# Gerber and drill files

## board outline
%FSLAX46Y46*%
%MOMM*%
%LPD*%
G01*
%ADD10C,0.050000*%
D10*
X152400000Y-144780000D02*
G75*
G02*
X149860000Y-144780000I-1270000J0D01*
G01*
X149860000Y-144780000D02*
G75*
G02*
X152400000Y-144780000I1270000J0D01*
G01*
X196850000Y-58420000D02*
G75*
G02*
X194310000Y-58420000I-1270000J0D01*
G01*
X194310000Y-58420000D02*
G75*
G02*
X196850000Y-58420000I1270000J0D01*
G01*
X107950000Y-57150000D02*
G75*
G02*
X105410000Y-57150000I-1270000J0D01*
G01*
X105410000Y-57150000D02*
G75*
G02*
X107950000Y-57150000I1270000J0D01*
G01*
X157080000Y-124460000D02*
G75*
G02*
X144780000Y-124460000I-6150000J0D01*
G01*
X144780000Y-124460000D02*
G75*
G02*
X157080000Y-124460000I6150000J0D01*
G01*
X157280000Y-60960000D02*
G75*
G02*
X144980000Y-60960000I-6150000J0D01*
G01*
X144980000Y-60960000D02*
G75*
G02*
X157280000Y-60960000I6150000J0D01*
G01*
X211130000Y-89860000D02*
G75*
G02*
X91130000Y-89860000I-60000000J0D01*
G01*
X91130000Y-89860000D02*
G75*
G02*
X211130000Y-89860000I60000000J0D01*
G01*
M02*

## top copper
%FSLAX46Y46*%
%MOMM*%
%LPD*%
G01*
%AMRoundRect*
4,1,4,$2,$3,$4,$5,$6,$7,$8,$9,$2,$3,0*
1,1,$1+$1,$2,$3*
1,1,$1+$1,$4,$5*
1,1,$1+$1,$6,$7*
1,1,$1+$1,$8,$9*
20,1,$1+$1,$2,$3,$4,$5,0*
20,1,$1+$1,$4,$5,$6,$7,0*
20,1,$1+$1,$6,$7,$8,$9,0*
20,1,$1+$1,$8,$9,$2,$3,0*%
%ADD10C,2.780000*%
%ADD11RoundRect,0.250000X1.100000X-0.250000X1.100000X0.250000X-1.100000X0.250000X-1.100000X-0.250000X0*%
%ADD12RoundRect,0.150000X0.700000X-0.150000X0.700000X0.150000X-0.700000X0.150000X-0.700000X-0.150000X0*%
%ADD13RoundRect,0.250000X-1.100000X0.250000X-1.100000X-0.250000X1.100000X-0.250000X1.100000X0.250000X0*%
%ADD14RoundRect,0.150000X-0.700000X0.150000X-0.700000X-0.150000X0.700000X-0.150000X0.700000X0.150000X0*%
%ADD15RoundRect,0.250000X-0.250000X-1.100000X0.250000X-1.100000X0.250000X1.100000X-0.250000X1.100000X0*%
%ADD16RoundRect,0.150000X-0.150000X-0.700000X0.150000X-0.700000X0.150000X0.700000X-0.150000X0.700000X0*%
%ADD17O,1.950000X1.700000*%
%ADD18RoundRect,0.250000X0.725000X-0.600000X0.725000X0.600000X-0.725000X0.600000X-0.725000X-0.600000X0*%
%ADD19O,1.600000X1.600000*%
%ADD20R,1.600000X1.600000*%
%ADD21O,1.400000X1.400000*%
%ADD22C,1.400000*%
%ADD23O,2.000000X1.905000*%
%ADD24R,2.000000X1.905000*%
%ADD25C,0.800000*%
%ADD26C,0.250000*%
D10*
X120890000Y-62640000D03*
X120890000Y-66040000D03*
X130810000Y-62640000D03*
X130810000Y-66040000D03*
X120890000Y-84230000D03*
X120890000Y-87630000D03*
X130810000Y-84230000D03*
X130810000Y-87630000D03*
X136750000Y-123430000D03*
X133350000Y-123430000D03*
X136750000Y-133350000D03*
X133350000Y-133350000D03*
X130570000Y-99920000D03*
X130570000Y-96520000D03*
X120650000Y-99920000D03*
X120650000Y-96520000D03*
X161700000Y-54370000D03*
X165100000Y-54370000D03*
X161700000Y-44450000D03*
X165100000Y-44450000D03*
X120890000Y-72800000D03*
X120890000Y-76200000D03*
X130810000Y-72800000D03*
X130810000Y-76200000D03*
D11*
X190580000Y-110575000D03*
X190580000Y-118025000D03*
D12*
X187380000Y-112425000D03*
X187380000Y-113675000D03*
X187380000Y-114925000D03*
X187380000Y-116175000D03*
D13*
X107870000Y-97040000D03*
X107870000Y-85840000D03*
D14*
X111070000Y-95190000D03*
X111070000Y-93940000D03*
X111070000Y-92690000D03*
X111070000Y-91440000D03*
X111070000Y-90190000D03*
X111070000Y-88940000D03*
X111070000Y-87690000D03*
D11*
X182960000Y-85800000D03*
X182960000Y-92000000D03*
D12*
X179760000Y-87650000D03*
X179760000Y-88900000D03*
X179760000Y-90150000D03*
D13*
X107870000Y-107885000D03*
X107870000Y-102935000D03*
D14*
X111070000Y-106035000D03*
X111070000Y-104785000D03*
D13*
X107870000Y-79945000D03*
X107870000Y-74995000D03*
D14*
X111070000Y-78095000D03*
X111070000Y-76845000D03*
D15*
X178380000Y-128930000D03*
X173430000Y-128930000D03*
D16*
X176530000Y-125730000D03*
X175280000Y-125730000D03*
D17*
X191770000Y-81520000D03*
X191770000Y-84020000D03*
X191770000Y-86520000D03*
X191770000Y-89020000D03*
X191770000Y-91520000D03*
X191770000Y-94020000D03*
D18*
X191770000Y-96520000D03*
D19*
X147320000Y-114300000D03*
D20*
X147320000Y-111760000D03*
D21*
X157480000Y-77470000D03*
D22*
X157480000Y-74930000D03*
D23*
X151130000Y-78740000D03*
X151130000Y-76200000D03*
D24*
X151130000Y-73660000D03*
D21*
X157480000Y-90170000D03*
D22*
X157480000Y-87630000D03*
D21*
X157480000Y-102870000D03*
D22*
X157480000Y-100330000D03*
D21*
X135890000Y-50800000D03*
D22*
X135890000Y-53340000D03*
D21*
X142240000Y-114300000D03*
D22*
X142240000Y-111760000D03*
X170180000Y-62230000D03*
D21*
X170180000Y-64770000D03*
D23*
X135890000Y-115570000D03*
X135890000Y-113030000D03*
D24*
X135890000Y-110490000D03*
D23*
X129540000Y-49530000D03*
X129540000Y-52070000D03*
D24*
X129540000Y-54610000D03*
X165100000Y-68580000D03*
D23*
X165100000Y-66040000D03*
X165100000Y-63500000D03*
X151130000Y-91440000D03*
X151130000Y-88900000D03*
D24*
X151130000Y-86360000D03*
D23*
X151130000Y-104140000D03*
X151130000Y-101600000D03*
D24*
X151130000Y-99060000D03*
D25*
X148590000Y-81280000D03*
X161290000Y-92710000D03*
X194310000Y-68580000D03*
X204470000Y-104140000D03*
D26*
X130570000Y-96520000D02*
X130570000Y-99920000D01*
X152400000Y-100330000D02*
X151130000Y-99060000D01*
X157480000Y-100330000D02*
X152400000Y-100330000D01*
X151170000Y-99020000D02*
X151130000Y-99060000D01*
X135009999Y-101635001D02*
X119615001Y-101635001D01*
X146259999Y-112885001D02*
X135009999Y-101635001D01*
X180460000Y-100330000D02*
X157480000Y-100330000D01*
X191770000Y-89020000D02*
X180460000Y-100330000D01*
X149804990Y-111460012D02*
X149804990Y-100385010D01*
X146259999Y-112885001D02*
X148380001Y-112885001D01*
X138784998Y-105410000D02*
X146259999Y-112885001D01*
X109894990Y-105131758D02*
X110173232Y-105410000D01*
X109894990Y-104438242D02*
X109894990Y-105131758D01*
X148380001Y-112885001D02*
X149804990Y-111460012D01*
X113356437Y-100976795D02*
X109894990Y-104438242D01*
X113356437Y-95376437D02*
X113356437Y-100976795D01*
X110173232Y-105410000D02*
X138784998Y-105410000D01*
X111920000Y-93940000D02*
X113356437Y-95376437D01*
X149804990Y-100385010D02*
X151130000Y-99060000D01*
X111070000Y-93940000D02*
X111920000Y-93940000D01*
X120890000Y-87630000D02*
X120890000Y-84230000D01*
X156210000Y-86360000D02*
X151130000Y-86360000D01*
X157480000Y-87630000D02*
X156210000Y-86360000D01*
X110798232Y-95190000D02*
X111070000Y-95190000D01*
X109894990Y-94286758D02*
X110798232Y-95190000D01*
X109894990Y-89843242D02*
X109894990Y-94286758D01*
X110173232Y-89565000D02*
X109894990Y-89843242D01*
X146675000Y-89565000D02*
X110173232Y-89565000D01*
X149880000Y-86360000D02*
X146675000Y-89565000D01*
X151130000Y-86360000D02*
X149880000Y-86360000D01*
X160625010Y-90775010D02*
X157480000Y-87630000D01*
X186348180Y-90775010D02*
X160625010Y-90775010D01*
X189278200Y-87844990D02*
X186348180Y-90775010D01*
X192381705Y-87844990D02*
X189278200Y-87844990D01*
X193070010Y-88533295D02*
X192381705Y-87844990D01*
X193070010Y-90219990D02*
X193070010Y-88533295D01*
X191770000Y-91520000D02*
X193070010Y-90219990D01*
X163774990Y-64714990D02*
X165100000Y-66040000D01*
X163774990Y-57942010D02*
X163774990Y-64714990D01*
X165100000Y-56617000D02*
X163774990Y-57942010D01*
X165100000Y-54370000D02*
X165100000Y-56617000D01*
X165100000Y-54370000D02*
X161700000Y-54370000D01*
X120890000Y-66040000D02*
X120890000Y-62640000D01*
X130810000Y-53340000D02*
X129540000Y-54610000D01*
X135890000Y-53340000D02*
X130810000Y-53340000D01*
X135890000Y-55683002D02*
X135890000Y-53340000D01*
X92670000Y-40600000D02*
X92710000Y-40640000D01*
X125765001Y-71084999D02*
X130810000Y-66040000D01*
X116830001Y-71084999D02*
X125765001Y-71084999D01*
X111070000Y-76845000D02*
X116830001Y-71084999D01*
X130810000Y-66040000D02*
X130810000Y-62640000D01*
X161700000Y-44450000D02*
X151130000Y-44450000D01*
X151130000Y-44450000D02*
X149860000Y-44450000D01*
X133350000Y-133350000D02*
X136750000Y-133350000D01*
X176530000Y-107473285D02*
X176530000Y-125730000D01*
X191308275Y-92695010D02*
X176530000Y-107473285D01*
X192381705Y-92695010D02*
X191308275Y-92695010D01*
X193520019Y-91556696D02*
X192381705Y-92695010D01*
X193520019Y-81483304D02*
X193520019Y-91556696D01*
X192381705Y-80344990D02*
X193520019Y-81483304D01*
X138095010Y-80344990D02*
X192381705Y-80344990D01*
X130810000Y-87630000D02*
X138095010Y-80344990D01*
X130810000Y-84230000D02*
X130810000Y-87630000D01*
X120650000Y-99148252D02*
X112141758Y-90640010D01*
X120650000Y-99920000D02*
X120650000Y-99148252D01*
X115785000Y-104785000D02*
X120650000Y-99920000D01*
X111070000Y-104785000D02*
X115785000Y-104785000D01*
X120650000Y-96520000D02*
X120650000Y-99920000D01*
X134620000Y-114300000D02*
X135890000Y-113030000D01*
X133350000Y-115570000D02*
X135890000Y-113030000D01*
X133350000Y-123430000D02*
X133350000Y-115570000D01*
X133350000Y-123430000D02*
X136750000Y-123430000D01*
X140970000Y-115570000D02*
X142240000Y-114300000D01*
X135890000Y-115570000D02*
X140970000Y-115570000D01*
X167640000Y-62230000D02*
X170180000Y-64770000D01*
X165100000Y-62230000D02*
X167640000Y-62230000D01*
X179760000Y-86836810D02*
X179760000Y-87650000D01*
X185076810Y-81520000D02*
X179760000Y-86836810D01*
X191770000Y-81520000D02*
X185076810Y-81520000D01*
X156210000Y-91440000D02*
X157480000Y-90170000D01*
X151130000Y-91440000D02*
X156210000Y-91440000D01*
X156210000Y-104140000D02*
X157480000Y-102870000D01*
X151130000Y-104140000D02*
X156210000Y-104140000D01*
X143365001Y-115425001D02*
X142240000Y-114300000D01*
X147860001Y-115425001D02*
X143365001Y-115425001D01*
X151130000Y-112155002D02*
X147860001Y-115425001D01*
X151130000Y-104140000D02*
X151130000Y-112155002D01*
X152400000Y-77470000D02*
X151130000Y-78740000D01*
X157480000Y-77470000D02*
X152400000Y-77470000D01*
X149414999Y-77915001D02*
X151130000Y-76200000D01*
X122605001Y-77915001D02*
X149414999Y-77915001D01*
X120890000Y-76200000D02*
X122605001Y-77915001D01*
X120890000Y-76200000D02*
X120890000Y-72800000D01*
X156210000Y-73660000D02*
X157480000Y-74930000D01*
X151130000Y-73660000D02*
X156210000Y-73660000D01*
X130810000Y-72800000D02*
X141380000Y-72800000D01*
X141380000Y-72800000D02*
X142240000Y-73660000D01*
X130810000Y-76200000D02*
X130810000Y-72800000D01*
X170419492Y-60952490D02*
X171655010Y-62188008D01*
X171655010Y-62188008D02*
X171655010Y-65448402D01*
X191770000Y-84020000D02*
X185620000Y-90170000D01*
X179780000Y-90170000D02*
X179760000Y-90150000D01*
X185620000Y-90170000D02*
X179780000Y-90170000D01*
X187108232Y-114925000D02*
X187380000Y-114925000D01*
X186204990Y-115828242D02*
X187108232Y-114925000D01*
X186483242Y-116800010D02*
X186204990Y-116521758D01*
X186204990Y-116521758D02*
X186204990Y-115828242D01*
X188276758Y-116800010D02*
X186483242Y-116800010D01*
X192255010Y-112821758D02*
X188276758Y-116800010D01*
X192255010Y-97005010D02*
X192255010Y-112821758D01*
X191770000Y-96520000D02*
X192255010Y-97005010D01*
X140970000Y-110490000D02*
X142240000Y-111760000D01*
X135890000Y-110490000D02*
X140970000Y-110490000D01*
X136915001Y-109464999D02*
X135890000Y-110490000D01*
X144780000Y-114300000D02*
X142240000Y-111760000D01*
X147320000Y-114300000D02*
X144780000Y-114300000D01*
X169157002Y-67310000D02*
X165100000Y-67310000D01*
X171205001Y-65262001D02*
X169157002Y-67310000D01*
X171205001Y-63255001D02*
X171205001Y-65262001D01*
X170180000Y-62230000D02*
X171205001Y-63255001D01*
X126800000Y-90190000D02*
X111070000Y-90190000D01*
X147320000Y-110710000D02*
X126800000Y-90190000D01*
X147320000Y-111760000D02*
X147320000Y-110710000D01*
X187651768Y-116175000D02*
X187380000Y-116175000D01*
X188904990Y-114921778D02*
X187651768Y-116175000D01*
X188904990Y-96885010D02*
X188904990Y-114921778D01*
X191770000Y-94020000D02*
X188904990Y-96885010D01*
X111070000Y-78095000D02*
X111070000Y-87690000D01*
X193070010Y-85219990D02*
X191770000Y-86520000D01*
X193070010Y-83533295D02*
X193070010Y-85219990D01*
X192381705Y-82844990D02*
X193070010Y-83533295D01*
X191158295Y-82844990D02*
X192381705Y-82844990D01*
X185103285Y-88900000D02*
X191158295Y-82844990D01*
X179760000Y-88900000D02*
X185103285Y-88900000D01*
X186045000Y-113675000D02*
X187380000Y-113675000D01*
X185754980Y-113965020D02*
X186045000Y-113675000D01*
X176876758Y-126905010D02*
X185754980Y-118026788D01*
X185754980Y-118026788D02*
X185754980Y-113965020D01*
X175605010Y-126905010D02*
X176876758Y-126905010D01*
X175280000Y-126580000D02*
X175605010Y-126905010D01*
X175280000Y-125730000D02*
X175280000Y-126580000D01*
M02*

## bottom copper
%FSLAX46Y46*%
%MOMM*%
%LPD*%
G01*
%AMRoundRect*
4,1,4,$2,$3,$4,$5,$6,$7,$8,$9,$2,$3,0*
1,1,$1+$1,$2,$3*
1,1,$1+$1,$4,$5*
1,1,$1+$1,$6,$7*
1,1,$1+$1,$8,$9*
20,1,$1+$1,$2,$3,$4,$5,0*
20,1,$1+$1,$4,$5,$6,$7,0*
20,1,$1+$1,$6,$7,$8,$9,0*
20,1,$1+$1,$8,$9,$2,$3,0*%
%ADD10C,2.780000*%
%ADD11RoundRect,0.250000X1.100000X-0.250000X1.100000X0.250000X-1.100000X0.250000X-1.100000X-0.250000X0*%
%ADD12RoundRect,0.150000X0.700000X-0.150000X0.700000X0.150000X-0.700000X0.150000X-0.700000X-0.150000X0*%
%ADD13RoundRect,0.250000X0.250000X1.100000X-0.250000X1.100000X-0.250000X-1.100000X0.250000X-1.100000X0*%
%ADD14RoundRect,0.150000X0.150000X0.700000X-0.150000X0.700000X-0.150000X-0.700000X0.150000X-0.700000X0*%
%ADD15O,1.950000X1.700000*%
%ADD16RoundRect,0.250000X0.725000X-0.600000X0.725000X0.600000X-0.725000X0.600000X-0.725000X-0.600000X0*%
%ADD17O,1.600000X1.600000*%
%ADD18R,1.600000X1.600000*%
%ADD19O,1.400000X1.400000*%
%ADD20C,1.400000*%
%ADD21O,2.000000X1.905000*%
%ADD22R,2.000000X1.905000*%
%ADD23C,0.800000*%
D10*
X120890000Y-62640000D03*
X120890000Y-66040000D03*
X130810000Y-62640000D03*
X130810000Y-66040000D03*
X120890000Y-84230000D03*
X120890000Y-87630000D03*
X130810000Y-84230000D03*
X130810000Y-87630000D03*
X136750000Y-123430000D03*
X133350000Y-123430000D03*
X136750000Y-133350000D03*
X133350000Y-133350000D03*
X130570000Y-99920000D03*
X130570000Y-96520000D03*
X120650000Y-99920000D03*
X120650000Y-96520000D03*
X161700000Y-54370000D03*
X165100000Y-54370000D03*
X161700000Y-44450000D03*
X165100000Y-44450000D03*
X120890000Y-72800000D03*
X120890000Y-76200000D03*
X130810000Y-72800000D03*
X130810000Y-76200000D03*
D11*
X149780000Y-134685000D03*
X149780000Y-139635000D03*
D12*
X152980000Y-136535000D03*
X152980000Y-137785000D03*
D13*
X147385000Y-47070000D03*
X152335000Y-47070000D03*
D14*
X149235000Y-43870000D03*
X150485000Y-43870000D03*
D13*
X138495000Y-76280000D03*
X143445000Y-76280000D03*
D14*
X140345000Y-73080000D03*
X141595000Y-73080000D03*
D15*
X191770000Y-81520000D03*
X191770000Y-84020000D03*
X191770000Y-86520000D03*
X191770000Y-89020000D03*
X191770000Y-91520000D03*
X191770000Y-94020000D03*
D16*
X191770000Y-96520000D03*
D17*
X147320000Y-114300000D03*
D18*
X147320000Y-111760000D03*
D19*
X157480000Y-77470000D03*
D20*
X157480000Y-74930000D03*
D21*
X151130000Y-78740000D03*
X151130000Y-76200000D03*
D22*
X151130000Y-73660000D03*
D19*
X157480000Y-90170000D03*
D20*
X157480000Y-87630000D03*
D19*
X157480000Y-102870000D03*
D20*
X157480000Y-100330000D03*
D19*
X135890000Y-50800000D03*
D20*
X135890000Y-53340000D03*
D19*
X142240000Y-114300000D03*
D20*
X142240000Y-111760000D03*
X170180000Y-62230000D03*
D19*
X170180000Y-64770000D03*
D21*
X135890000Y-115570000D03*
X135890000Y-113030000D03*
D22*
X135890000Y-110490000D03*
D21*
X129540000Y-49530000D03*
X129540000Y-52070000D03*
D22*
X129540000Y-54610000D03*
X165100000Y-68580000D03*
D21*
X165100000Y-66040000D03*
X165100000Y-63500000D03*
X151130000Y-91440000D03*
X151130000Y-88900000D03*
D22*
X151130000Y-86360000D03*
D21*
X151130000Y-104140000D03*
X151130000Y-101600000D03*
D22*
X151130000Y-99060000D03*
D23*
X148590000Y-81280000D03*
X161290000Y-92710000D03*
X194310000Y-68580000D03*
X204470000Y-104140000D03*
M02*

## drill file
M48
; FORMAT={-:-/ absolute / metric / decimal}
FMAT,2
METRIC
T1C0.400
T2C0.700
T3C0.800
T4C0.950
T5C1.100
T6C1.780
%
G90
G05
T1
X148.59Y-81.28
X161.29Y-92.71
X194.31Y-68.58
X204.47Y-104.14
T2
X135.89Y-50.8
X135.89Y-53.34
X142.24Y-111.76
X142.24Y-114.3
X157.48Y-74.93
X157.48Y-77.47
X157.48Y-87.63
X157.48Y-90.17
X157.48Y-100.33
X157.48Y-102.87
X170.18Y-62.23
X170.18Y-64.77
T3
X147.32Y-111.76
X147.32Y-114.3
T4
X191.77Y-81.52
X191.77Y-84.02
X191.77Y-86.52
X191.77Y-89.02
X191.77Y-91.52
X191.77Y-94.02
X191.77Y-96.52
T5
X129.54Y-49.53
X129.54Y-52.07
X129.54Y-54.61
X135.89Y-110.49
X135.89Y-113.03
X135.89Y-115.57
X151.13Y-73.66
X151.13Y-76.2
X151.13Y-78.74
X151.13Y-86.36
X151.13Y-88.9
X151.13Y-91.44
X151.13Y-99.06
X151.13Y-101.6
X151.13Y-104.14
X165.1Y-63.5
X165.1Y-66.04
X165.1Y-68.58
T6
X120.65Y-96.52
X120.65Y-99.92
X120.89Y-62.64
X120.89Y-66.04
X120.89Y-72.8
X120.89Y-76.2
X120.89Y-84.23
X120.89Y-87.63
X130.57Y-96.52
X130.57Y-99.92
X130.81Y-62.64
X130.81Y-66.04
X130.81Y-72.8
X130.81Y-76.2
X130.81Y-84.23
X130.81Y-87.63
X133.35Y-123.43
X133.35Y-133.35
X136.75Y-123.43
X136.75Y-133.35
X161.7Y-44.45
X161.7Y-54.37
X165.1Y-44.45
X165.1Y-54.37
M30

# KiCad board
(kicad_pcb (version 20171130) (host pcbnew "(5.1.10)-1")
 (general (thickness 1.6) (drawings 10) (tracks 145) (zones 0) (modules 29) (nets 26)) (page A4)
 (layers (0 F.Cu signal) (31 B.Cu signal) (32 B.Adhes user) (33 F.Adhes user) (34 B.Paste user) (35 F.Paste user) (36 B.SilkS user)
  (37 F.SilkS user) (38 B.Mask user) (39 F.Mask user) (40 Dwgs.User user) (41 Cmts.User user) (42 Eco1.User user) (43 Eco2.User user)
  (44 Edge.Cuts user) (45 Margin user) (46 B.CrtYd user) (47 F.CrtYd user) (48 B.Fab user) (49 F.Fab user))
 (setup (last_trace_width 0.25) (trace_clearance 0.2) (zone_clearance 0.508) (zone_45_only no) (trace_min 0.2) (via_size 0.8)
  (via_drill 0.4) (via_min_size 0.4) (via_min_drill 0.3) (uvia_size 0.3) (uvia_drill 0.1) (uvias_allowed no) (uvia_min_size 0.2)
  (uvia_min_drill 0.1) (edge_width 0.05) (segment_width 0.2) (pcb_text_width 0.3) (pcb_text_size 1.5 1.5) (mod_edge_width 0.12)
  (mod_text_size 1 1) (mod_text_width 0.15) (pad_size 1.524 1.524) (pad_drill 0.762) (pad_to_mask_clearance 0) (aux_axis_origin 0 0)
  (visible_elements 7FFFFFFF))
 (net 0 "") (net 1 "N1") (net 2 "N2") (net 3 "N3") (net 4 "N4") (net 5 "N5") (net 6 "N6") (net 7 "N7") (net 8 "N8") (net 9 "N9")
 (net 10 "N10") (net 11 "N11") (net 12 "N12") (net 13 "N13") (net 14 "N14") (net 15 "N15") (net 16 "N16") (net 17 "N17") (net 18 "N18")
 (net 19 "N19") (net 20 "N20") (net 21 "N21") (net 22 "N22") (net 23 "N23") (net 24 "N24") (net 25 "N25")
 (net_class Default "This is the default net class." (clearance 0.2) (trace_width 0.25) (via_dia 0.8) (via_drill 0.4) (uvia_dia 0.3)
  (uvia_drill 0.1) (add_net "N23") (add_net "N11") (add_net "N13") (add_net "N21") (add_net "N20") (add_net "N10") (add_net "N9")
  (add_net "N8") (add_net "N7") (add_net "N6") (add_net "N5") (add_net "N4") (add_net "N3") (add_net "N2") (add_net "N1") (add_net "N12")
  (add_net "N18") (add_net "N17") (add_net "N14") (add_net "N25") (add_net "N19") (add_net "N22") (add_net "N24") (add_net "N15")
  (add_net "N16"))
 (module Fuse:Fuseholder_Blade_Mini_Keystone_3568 (layer F.Cu) (at 130.81 66.04 180)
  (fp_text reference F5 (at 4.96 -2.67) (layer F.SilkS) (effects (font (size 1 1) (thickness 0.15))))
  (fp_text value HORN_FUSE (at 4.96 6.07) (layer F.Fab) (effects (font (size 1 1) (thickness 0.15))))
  (pad 2 thru_hole circle (at 9.92 3.4 180) (size 2.78 2.78) (drill 1.78) (layers *.Cu *.Mask) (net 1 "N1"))
  (pad 2 thru_hole circle (at 9.92 0 180) (size 2.78 2.78) (drill 1.78) (layers *.Cu *.Mask) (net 1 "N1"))
  (pad 1 thru_hole circle (at 0 3.4 180) (size 2.78 2.78) (drill 1.78) (layers *.Cu *.Mask) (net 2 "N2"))
  (pad 1 thru_hole circle (at 0 0 180) (size 2.78 2.78) (drill 1.78) (layers *.Cu *.Mask) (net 2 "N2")))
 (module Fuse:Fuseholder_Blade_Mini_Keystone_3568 (layer F.Cu) (at 130.81 87.63 180)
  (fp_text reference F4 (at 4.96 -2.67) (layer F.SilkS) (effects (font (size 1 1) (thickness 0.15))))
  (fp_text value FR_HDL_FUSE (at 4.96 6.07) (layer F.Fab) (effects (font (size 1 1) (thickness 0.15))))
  (pad 2 thru_hole circle (at 9.92 3.4 180) (size 2.78 2.78) (drill 1.78) (layers *.Cu *.Mask) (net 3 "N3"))
  (pad 2 thru_hole circle (at 9.92 0 180) (size 2.78 2.78) (drill 1.78) (layers *.Cu *.Mask) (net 3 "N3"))
  (pad 1 thru_hole circle (at 0 3.4 180) (size 2.78 2.78) (drill 1.78) (layers *.Cu *.Mask) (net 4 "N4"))
  (pad 1 thru_hole circle (at 0 0 180) (size 2.78 2.78) (drill 1.78) (layers *.Cu *.Mask) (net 4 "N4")))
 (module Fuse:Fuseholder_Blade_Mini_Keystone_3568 (layer F.Cu) (at 133.35 133.35 90)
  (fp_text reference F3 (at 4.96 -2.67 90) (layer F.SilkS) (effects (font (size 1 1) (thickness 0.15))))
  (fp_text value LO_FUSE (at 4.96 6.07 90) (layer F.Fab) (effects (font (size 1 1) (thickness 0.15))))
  (pad 2 thru_hole circle (at 9.92 3.4 90) (size 2.78 2.78) (drill 1.78) (layers *.Cu *.Mask) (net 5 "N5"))
  (pad 2 thru_hole circle (at 9.92 0 90) (size 2.78 2.78) (drill 1.78) (layers *.Cu *.Mask) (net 5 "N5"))
  (pad 1 thru_hole circle (at 0 3.4 90) (size 2.78 2.78) (drill 1.78) (layers *.Cu *.Mask) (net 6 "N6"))
  (pad 1 thru_hole circle (at 0 0 90) (size 2.78 2.78) (drill 1.78) (layers *.Cu *.Mask) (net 6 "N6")))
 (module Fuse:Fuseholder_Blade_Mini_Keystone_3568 (layer F.Cu) (at 120.65 96.52)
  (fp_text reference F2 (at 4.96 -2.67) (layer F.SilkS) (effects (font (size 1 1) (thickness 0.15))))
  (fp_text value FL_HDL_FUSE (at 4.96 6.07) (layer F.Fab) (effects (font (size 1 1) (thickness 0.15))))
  (pad 2 thru_hole circle (at 9.92 3.4) (size 2.78 2.78) (drill 1.78) (layers *.Cu *.Mask) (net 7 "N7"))
  (pad 2 thru_hole circle (at 9.92 0) (size 2.78 2.78) (drill 1.78) (layers *.Cu *.Mask) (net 7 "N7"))
  (pad 1 thru_hole circle (at 0 3.4) (size 2.78 2.78) (drill 1.78) (layers *.Cu *.Mask) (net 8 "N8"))
  (pad 1 thru_hole circle (at 0 0) (size 2.78 2.78) (drill 1.78) (layers *.Cu *.Mask) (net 8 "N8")))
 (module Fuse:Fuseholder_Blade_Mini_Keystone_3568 (layer F.Cu) (at 165.1 44.45 270)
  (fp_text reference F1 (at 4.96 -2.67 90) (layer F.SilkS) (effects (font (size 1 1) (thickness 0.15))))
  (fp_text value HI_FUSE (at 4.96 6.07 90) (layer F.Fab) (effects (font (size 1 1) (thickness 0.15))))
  (pad 2 thru_hole circle (at 9.92 3.4 270) (size 2.78 2.78) (drill 1.78) (layers *.Cu *.Mask) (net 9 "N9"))
  (pad 2 thru_hole circle (at 9.92 0 270) (size 2.78 2.78) (drill 1.78) (layers *.Cu *.Mask) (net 9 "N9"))
  (pad 1 thru_hole circle (at 0 3.4 270) (size 2.78 2.78) (drill 1.78) (layers *.Cu *.Mask) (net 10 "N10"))
  (pad 1 thru_hole circle (at 0 0 270) (size 2.78 2.78) (drill 1.78) (layers *.Cu *.Mask) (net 10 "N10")))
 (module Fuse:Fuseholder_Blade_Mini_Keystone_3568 (layer F.Cu) (at 130.81 76.2 180)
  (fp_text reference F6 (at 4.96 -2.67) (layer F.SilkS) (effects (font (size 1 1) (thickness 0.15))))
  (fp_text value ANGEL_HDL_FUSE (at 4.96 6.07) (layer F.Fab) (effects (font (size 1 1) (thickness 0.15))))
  (pad 2 thru_hole circle (at 9.92 3.4 180) (size 2.78 2.78) (drill 1.78) (layers *.Cu *.Mask) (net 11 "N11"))
  (pad 2 thru_hole circle (at 9.92 0 180) (size 2.78 2.78) (drill 1.78) (layers *.Cu *.Mask) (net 11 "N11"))
  (pad 1 thru_hole circle (at 0 3.4 180) (size 2.78 2.78) (drill 1.78) (layers *.Cu *.Mask) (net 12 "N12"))
  (pad 1 thru_hole circle (at 0 0 180) (size 2.78 2.78) (drill 1.78) (layers *.Cu *.Mask) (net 12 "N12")))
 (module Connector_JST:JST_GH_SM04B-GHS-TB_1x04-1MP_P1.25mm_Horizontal (layer F.Cu) (at 189.23 114.3 90)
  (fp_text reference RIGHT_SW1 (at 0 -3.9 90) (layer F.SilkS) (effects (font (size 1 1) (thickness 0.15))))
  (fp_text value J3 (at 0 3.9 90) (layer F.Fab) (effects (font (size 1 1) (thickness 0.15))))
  (pad MP smd roundrect (at 3.725 1.35 90) (size 1 2.7) (layers F.Cu F.Paste F.Mask) (roundrect_rratio 0.25))
  (pad MP smd roundrect (at -3.725 1.35 90) (size 1 2.7) (layers F.Cu F.Paste F.Mask) (roundrect_rratio 0.25))
  (pad 4 smd roundrect (at 1.875 -1.85 90) (size 0.6 1.7) (layers F.Cu F.Paste F.Mask) (roundrect_rratio 0.25) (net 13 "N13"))
  (pad 3 smd roundrect (at 0.625 -1.85 90) (size 0.6 1.7) (layers F.Cu F.Paste F.Mask) (roundrect_rratio 0.25) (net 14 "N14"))
  (pad 2 smd roundrect (at -0.625 -1.85 90) (size 0.6 1.7) (layers F.Cu F.Paste F.Mask) (roundrect_rratio 0.25) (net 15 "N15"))
  (pad 1 smd roundrect (at -1.875 -1.85 90) (size 0.6 1.7) (layers F.Cu F.Paste F.Mask) (roundrect_rratio 0.25) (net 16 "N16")))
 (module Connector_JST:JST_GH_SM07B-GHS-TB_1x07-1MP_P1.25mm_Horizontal (layer F.Cu) (at 109.22 91.44 270)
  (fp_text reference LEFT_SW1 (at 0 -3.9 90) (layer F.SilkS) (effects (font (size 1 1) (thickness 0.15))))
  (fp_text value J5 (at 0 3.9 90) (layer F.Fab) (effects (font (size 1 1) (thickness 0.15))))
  (pad MP smd roundrect (at 5.6 1.35 270) (size 1 2.7) (layers F.Cu F.Paste F.Mask) (roundrect_rratio 0.25))
  (pad MP smd roundrect (at -5.6 1.35 270) (size 1 2.7) (layers F.Cu F.Paste F.Mask) (roundrect_rratio 0.25))
  (pad 7 smd roundrect (at 3.75 -1.85 270) (size 0.6 1.7) (layers F.Cu F.Paste F.Mask) (roundrect_rratio 0.25) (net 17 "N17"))
  (pad 6 smd roundrect (at 2.5 -1.85 270) (size 0.6 1.7) (layers F.Cu F.Paste F.Mask) (roundrect_rratio 0.25) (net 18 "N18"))
  (pad 5 smd roundrect (at 1.25 -1.85 270) (size 0.6 1.7) (layers F.Cu F.Paste F.Mask) (roundrect_rratio 0.25) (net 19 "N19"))
  (pad 4 smd roundrect (at 0 -1.85 270) (size 0.6 1.7) (layers F.Cu F.Paste F.Mask) (roundrect_rratio 0.25) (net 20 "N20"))
  (pad 3 smd roundrect (at -1.25 -1.85 270) (size 0.6 1.7) (layers F.Cu F.Paste F.Mask) (roundrect_rratio 0.25) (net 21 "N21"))
  (pad 2 smd roundrect (at -2.5 -1.85 270) (size 0.6 1.7) (layers F.Cu F.Paste F.Mask) (roundrect_rratio 0.25) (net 13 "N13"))
  (pad 1 smd roundrect (at -3.75 -1.85 270) (size 0.6 1.7) (layers F.Cu F.Paste F.Mask) (roundrect_rratio 0.25) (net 14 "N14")))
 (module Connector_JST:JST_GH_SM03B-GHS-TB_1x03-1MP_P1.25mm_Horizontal (layer F.Cu) (at 181.61 88.9 90)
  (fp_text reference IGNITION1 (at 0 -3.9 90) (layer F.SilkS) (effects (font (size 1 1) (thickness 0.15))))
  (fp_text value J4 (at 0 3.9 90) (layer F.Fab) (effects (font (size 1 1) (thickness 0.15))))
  (pad MP smd roundrect (at 3.1 1.35 90) (size 1 2.7) (layers F.Cu F.Paste F.Mask) (roundrect_rratio 0.25))
  (pad MP smd roundrect (at -3.1 1.35 90) (size 1 2.7) (layers F.Cu F.Paste F.Mask) (roundrect_rratio 0.25))
  (pad 3 smd roundrect (at 1.25 -1.85 90) (size 0.6 1.7) (layers F.Cu F.Paste F.Mask) (roundrect_rratio 0.25) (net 13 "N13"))
  (pad 2 smd roundrect (at 0 -1.85 90) (size 0.6 1.7) (layers F.Cu F.Paste F.Mask) (roundrect_rratio 0.25) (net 14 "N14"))
  (pad 1 smd roundrect (at -1.25 -1.85 90) (size 0.6 1.7) (layers F.Cu F.Paste F.Mask) (roundrect_rratio 0.25) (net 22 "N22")))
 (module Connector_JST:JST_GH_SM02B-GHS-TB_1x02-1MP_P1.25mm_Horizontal (layer F.Cu) (at 109.22 105.41 270)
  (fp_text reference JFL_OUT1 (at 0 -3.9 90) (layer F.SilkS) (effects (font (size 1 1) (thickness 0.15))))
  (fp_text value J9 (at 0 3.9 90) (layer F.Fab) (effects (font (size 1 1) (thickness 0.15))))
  (pad MP smd roundrect (at 2.475 1.35 270) (size 1 2.7) (layers F.Cu F.Paste F.Mask) (roundrect_rratio 0.25))
  (pad MP smd roundrect (at -2.475 1.35 270) (size 1 2.7) (layers F.Cu F.Paste F.Mask) (roundrect_rratio 0.25))
  (pad 2 smd roundrect (at 0.625 -1.85 270) (size 0.6 1.7) (layers F.Cu F.Paste F.Mask) (roundrect_rratio 0.25) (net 14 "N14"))
  (pad 1 smd roundrect (at -0.625 -1.85 270) (size 0.6 1.7) (layers F.Cu F.Paste F.Mask) (roundrect_rratio 0.25) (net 8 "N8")))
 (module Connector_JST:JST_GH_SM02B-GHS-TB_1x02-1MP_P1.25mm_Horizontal (layer B.Cu) (at 151.13 137.16 90)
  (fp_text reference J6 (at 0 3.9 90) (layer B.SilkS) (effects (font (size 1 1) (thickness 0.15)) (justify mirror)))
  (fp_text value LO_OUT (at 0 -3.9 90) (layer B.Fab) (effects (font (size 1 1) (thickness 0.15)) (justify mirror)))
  (pad MP smd roundrect (at 2.475 -1.35 90) (size 1 2.7) (layers B.Cu B.Paste B.Mask) (roundrect_rratio 0.25))
  (pad MP smd roundrect (at -2.475 -1.35 90) (size 1 2.7) (layers B.Cu B.Paste B.Mask) (roundrect_rratio 0.25))
  (pad 2 smd roundrect (at 0.625 1.85 90) (size 0.6 1.7) (layers B.Cu B.Paste B.Mask) (roundrect_rratio 0.25) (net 14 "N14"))
  (pad 1 smd roundrect (at -0.625 1.85 90) (size 0.6 1.7) (layers B.Cu B.Paste B.Mask) (roundrect_rratio 0.25) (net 6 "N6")))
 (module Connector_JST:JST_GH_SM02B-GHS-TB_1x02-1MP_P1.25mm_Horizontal (layer B.Cu) (at 149.86 45.72 180)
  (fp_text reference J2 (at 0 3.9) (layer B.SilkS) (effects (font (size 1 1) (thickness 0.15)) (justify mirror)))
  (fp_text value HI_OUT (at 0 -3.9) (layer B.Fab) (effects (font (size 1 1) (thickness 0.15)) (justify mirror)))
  (pad MP smd roundrect (at 2.475 -1.35 180) (size 1 2.7) (layers B.Cu B.Paste B.Mask) (roundrect_rratio 0.25))
  (pad MP smd roundrect (at -2.475 -1.35 180) (size 1 2.7) (layers B.Cu B.Paste B.Mask) (roundrect_rratio 0.25))
  (pad 2 smd roundrect (at 0.625 1.85 180) (size 0.6 1.7) (layers B.Cu B.Paste B.Mask) (roundrect_rratio 0.25) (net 14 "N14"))
  (pad 1 smd roundrect (at -0.625 1.85 180) (size 0.6 1.7) (layers B.Cu B.Paste B.Mask) (roundrect_rratio 0.25) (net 10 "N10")))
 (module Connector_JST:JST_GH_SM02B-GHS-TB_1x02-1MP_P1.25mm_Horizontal (layer F.Cu) (at 109.22 77.47 270)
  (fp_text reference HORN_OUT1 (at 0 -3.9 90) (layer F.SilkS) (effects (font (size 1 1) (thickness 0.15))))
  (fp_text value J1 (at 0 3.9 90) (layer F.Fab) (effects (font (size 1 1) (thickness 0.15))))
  (pad MP smd roundrect (at 2.475 1.35 270) (size 1 2.7) (layers F.Cu F.Paste F.Mask) (roundrect_rratio 0.25))
  (pad MP smd roundrect (at -2.475 1.35 270) (size 1 2.7) (layers F.Cu F.Paste F.Mask) (roundrect_rratio 0.25))
  (pad 2 smd roundrect (at 0.625 -1.85 270) (size 0.6 1.7) (layers F.Cu F.Paste F.Mask) (roundrect_rratio 0.25) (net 14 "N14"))
  (pad 1 smd roundrect (at -0.625 -1.85 270) (size 0.6 1.7) (layers F.Cu F.Paste F.Mask) (roundrect_rratio 0.25) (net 2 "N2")))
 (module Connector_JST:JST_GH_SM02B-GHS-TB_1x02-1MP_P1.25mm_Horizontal (layer B.Cu) (at 140.97 74.93 180)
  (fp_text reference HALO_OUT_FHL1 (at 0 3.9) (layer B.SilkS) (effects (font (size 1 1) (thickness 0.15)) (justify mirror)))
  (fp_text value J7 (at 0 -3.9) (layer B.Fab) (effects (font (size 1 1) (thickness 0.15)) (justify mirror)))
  (pad MP smd roundrect (at 2.475 -1.35 180) (size 1 2.7) (layers B.Cu B.Paste B.Mask) (roundrect_rratio 0.25))
  (pad MP smd roundrect (at -2.475 -1.35 180) (size 1 2.7) (layers B.Cu B.Paste B.Mask) (roundrect_rratio 0.25))
  (pad 2 smd roundrect (at 0.625 1.85 180) (size 0.6 1.7) (layers B.Cu B.Paste B.Mask) (roundrect_rratio 0.25) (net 14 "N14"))
  (pad 1 smd roundrect (at -0.625 1.85 180) (size 0.6 1.7) (layers B.Cu B.Paste B.Mask) (roundrect_rratio 0.25) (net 12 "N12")))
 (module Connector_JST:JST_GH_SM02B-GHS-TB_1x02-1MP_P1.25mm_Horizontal (layer F.Cu) (at 175.905 127.58)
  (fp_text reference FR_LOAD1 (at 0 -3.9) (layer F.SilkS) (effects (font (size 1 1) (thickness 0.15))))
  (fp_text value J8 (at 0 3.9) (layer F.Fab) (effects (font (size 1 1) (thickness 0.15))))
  (pad MP smd roundrect (at 2.475 1.35) (size 1 2.7) (layers F.Cu F.Paste F.Mask) (roundrect_rratio 0.25))
  (pad MP smd roundrect (at -2.475 1.35) (size 1 2.7) (layers F.Cu F.Paste F.Mask) (roundrect_rratio 0.25))
  (pad 2 smd roundrect (at 0.625 -1.85) (size 0.6 1.7) (layers F.Cu F.Paste F.Mask) (roundrect_rratio 0.25) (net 4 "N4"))
  (pad 1 smd roundrect (at -0.625 -1.85) (size 0.6 1.7) (layers F.Cu F.Paste F.Mask) (roundrect_rratio 0.25) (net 14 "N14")))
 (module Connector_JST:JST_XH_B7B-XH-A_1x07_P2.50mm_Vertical (layer F.Cu) (at 191.77 96.52 90)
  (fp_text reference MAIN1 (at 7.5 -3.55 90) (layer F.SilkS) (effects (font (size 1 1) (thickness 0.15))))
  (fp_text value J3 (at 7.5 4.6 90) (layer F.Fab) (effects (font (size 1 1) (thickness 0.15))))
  (pad 7 thru_hole oval (at 15 0 90) (size 1.7 1.95) (drill 0.95) (layers *.Cu *.Mask) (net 13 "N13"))
  (pad 6 thru_hole oval (at 12.5 0 90) (size 1.7 1.95) (drill 0.95) (layers *.Cu *.Mask) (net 22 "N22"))
  (pad 5 thru_hole oval (at 10 0 90) (size 1.7 1.95) (drill 0.95) (layers *.Cu *.Mask) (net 14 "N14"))
  (pad 4 thru_hole oval (at 7.5 0 90) (size 1.7 1.95) (drill 0.95) (layers *.Cu *.Mask) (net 18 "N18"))
  (pad 3 thru_hole oval (at 5 0 90) (size 1.7 1.95) (drill 0.95) (layers *.Cu *.Mask) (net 17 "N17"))
  (pad 2 thru_hole oval (at 2.5 0 90) (size 1.7 1.95) (drill 0.95) (layers *.Cu *.Mask) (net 16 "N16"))
  (pad 1 thru_hole roundrect (at 0 0 90) (size 1.7 1.95) (drill 0.95) (layers *.Cu *.Mask) (roundrect_rratio 0.147059) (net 15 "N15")))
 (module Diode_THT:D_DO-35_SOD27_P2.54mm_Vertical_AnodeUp (layer F.Cu) (at 147.32 111.76 270)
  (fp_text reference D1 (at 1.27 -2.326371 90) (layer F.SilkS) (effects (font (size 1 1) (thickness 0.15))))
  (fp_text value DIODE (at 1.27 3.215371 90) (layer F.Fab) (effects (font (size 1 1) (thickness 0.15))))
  (pad 2 thru_hole oval (at 2.54 0 270) (size 1.6 1.6) (drill 0.8) (layers *.Cu *.Mask) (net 20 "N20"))
  (pad 1 thru_hole rect (at 0 0 270) (size 1.6 1.6) (drill 0.8) (layers *.Cu *.Mask) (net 21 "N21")))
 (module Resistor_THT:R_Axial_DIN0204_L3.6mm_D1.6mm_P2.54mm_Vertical (layer F.Cu) (at 157.48 74.93 270)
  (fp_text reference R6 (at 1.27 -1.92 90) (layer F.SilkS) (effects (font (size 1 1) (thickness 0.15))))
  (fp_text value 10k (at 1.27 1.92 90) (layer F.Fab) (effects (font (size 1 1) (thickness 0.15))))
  (pad 2 thru_hole oval (at 2.54 0 270) (size 1.4 1.4) (drill 0.7) (layers *.Cu *.Mask) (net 13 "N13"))
  (pad 1 thru_hole circle (at 0 0 270) (size 1.4 1.4) (drill 0.7) (layers *.Cu *.Mask) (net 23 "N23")))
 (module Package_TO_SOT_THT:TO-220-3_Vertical (layer F.Cu) (at 151.13 73.66 270)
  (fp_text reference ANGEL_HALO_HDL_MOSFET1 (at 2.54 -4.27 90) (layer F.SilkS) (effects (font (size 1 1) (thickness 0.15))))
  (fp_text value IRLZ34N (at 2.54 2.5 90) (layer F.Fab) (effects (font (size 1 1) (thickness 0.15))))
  (pad 3 thru_hole oval (at 5.08 0 270) (size 1.905 2) (drill 1.1) (layers *.Cu *.Mask) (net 13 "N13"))
  (pad 2 thru_hole oval (at 2.54 0 270) (size 1.905 2) (drill 1.1) (layers *.Cu *.Mask) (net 11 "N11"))
  (pad 1 thru_hole rect (at 0 0 270) (size 1.905 2) (drill 1.1) (layers *.Cu *.Mask) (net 23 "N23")))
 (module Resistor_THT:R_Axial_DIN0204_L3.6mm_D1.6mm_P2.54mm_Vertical (layer F.Cu) (at 157.48 87.63 270)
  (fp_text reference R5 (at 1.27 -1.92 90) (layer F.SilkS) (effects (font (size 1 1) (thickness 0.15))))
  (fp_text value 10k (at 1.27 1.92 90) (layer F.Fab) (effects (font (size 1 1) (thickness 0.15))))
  (pad 2 thru_hole oval (at 2.54 0 270) (size 1.4 1.4) (drill 0.7) (layers *.Cu *.Mask) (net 13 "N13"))
  (pad 1 thru_hole circle (at 0 0 270) (size 1.4 1.4) (drill 0.7) (layers *.Cu *.Mask) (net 17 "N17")))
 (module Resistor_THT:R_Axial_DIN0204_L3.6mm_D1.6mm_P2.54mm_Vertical (layer F.Cu) (at 157.48 100.33 270)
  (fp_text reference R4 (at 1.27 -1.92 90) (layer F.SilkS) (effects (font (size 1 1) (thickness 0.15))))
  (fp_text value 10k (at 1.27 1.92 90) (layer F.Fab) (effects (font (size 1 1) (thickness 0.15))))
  (pad 2 thru_hole oval (at 2.54 0 270) (size 1.4 1.4) (drill 0.7) (layers *.Cu *.Mask) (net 13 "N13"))
  (pad 1 thru_hole circle (at 0 0 270) (size 1.4 1.4) (drill 0.7) (layers *.Cu *.Mask) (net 18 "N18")))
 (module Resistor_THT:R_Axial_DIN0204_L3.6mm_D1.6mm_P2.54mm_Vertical (layer F.Cu) (at 135.89 53.34 90)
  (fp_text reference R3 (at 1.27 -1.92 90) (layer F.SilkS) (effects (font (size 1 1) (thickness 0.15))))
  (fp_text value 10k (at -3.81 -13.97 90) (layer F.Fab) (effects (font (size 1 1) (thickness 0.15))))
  (pad 2 thru_hole oval (at 2.54 0 90) (size 1.4 1.4) (drill 0.7) (layers *.Cu *.Mask) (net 13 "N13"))
  (pad 1 thru_hole circle (at 0 0 90) (size 1.4 1.4) (drill 0.7) (layers *.Cu *.Mask) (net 19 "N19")))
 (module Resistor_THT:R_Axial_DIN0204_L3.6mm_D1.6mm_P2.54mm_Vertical (layer F.Cu) (at 142.24 111.76 270)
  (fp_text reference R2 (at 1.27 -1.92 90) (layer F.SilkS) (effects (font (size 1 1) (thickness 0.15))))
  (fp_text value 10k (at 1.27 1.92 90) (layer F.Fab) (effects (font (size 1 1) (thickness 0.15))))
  (pad 2 thru_hole oval (at 2.54 0 270) (size 1.4 1.4) (drill 0.7) (layers *.Cu *.Mask) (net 13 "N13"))
  (pad 1 thru_hole circle (at 0 0 270) (size 1.4 1.4) (drill 0.7) (layers *.Cu *.Mask) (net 20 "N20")))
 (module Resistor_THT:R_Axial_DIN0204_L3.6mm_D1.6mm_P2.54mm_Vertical (layer F.Cu) (at 170.18 62.23 270)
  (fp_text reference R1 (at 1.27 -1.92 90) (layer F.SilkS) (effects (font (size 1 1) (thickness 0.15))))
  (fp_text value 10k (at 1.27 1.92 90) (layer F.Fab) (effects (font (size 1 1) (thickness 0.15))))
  (pad 1 thru_hole circle (at 0 0 270) (size 1.4 1.4) (drill 0.7) (layers *.Cu *.Mask) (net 21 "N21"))
  (pad 2 thru_hole oval (at 2.54 0 270) (size 1.4 1.4) (drill 0.7) (layers *.Cu *.Mask) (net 13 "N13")))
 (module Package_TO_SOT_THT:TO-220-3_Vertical (layer F.Cu) (at 135.89 110.49 270)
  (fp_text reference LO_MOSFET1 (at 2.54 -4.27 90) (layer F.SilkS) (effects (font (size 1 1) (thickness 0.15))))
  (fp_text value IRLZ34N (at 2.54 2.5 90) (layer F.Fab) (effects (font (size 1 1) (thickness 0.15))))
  (pad 3 thru_hole oval (at 5.08 0 270) (size 1.905 2) (drill 1.1) (layers *.Cu *.Mask) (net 13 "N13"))
  (pad 2 thru_hole oval (at 2.54 0 270) (size 1.905 2) (drill 1.1) (layers *.Cu *.Mask) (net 5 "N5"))
  (pad 1 thru_hole rect (at 0 0 270) (size 1.905 2) (drill 1.1) (layers *.Cu *.Mask) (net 20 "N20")))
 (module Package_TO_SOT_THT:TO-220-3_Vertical (layer F.Cu) (at 129.54 54.61 90)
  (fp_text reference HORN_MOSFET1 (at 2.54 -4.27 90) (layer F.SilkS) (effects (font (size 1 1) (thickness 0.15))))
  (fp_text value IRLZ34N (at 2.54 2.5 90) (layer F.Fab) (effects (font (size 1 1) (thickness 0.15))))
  (pad 3 thru_hole oval (at 5.08 0 90) (size 1.905 2) (drill 1.1) (layers *.Cu *.Mask) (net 13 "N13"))
  (pad 2 thru_hole oval (at 2.54 0 90) (size 1.905 2) (drill 1.1) (layers *.Cu *.Mask) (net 1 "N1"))
  (pad 1 thru_hole rect (at 0 0 90) (size 1.905 2) (drill 1.1) (layers *.Cu *.Mask) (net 19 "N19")))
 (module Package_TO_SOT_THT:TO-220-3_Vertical (layer F.Cu) (at 165.1 68.58 90)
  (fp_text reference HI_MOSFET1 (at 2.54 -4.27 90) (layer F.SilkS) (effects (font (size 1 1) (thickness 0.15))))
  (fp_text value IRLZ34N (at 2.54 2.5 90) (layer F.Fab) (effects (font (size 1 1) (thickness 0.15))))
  (pad 1 thru_hole rect (at 0 0 90) (size 1.905 2) (drill 1.1) (layers *.Cu *.Mask) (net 21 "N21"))
  (pad 2 thru_hole oval (at 2.54 0 90) (size 1.905 2) (drill 1.1) (layers *.Cu *.Mask) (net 9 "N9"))
  (pad 3 thru_hole oval (at 5.08 0 90) (size 1.905 2) (drill 1.1) (layers *.Cu *.Mask) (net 13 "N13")))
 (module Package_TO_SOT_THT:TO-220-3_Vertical (layer F.Cu) (at 151.13 86.36 270)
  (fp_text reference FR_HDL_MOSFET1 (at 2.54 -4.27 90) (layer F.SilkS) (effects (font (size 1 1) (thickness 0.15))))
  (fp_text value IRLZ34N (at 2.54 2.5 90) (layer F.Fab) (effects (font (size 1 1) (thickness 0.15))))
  (pad 3 thru_hole oval (at 5.08 0 270) (size 1.905 2) (drill 1.1) (layers *.Cu *.Mask) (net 13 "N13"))
  (pad 2 thru_hole oval (at 2.54 0 270) (size 1.905 2) (drill 1.1) (layers *.Cu *.Mask) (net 3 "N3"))
  (pad 1 thru_hole rect (at 0 0 270) (size 1.905 2) (drill 1.1) (layers *.Cu *.Mask) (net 17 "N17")))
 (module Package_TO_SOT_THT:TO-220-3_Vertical (layer F.Cu) (at 151.13 99.06 270)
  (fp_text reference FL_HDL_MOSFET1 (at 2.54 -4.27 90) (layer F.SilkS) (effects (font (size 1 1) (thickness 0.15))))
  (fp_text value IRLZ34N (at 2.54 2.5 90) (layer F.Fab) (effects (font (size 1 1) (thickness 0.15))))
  (pad 3 thru_hole oval (at 5.08 0 270) (size 1.905 2) (drill 1.1) (layers *.Cu *.Mask) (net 13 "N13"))
  (pad 2 thru_hole oval (at 2.54 0 270) (size 1.905 2) (drill 1.1) (layers *.Cu *.Mask) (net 7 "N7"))
  (pad 1 thru_hole rect (at 0 0 270) (size 1.905 2) (drill 1.1) (layers *.Cu *.Mask) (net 18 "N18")))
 (gr_circle (center 151.13 144.78) (end 152.4 144.78) (layer Edge.Cuts) (width 0.05))
 (gr_circle (center 195.58 58.42) (end 196.85 58.42) (layer Edge.Cuts) (width 0.05))
 (gr_circle (center 106.68 57.15) (end 106.68 58.42) (layer Edge.Cuts) (width 0.05))
 (gr_circle (center 150.93 124.46) (end 157.08 124.46) (layer Edge.Cuts) (width 0.05))
 (gr_circle (center 151.13 60.96) (end 157.28 60.96) (layer Edge.Cuts) (width 0.05))
 (gr_circle (center 151.13 89.86) (end 211.13 89.86) (layer Edge.Cuts) (width 0.05))
 (via (at 148.59 81.28) (size 0.8) (drill 0.4) (layers F.Cu B.Cu) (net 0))
 (segment (start 130.57 96.52) (end 130.57 99.92) (width 0.25) (layer F.Cu) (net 7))
 (segment (start 152.4 100.33) (end 151.13 99.06) (width 0.25) (layer F.Cu) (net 18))
 (segment (start 157.48 100.33) (end 152.4 100.33) (width 0.25) (layer F.Cu) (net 18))
 (segment (start 151.17 99.02) (end 151.13 99.06) (width 0.25) (layer F.Cu) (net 18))
 (segment (start 135.009999 101.635001) (end 119.615001 101.635001) (width 0.25) (layer F.Cu) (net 18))
 (segment (start 146.259999 112.885001) (end 135.009999 101.635001) (width 0.25) (layer F.Cu) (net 18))
 (segment (start 180.46 100.33) (end 157.48 100.33) (width 0.25) (layer F.Cu) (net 18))
 (segment (start 191.77 89.02) (end 180.46 100.33) (width 0.25) (layer F.Cu) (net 18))
 (segment (start 149.80499 111.460012) (end 149.80499 100.38501) (width 0.25) (layer F.Cu) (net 18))
 (segment (start 146.259999 112.885001) (end 148.380001 112.885001) (width 0.25) (layer F.Cu) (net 18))
 (segment (start 138.784998 105.41) (end 146.259999 112.885001) (width 0.25) (layer F.Cu) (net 18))
 (segment (start 109.89499 105.131758) (end 110.173232 105.41) (width 0.25) (layer F.Cu) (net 18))
 (segment (start 109.89499 104.438242) (end 109.89499 105.131758) (width 0.25) (layer F.Cu) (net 18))
 (segment (start 148.380001 112.885001) (end 149.80499 111.460012) (width 0.25) (layer F.Cu) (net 18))
 (segment (start 113.356437 100.976795) (end 109.89499 104.438242) (width 0.25) (layer F.Cu) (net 18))
 (segment (start 113.356437 95.376437) (end 113.356437 100.976795) (width 0.25) (layer F.Cu) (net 18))
 (segment (start 110.173232 105.41) (end 138.784998 105.41) (width 0.25) (layer F.Cu) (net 18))
 (segment (start 111.92 93.94) (end 113.356437 95.376437) (width 0.25) (layer F.Cu) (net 18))
 (segment (start 149.80499 100.38501) (end 151.13 99.06) (width 0.25) (layer F.Cu) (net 18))
 (segment (start 111.07 93.94) (end 111.92 93.94) (width 0.25) (layer F.Cu) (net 18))
 (segment (start 120.89 87.63) (end 120.89 84.23) (width 0.25) (layer F.Cu) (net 3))
 (segment (start 156.21 86.36) (end 151.13 86.36) (width 0.25) (layer F.Cu) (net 17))
 (segment (start 157.48 87.63) (end 156.21 86.36) (width 0.25) (layer F.Cu) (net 17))
 (segment (start 110.798232 95.19) (end 111.07 95.19) (width 0.25) (layer F.Cu) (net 17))
 (segment (start 109.89499 94.286758) (end 110.798232 95.19) (width 0.25) (layer F.Cu) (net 17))
 (segment (start 109.89499 89.843242) (end 109.89499 94.286758) (width 0.25) (layer F.Cu) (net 17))
 (segment (start 110.173232 89.565) (end 109.89499 89.843242) (width 0.25) (layer F.Cu) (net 17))
 (segment (start 146.675 89.565) (end 110.173232 89.565) (width 0.25) (layer F.Cu) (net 17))
 (segment (start 149.88 86.36) (end 146.675 89.565) (width 0.25) (layer F.Cu) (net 17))
 (segment (start 151.13 86.36) (end 149.88 86.36) (width 0.25) (layer F.Cu) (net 17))
 (segment (start 160.62501 90.77501) (end 157.48 87.63) (width 0.25) (layer F.Cu) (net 17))
 (segment (start 186.34818 90.77501) (end 160.62501 90.77501) (width 0.25) (layer F.Cu) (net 17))
 (segment (start 189.2782 87.84499) (end 186.34818 90.77501) (width 0.25) (layer F.Cu) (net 17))
 (segment (start 192.381705 87.84499) (end 189.2782 87.84499) (width 0.25) (layer F.Cu) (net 17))
 (segment (start 193.07001 88.533295) (end 192.381705 87.84499) (width 0.25) (layer F.Cu) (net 17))
 (segment (start 193.07001 90.21999) (end 193.07001 88.533295) (width 0.25) (layer F.Cu) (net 17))
 (segment (start 191.77 91.52) (end 193.07001 90.21999) (width 0.25) (layer F.Cu) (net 17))
 (segment (start 163.77499 64.71499) (end 165.1 66.04) (width 0.25) (layer F.Cu) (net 9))
 (segment (start 163.77499 57.94201) (end 163.77499 64.71499) (width 0.25) (layer F.Cu) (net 9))
 (segment (start 165.1 56.617) (end 163.77499 57.94201) (width 0.25) (layer F.Cu) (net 9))
 (segment (start 165.1 54.37) (end 165.1 56.617) (width 0.25) (layer F.Cu) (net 9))
 (segment (start 165.1 54.37) (end 161.7 54.37) (width 0.25) (layer F.Cu) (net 9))
 (via (at 161.29 92.71) (size 0.8) (drill 0.4) (layers F.Cu B.Cu) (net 1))
 (segment (start 120.89 66.04) (end 120.89 62.64) (width 0.25) (layer F.Cu) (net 1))
 (segment (start 130.81 53.34) (end 129.54 54.61) (width 0.25) (layer F.Cu) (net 19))
 (segment (start 135.89 53.34) (end 130.81 53.34) (width 0.25) (layer F.Cu) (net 19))
 (segment (start 135.89 55.683002) (end 135.89 53.34) (width 0.25) (layer F.Cu) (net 19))
 (via (at 194.31 68.58) (size 0.8) (drill 0.4) (layers F.Cu B.Cu) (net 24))
 (segment (start 92.67 40.6) (end 92.71 40.64) (width 0.25) (layer F.Cu) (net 2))
 (segment (start 125.765001 71.084999) (end 130.81 66.04) (width 0.25) (layer F.Cu) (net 2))
 (segment (start 116.830001 71.084999) (end 125.765001 71.084999) (width 0.25) (layer F.Cu) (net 2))
 (segment (start 111.07 76.845) (end 116.830001 71.084999) (width 0.25) (layer F.Cu) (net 2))
 (segment (start 130.81 66.04) (end 130.81 62.64) (width 0.25) (layer F.Cu) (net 2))
 (segment (start 161.7 44.45) (end 151.13 44.45) (width 0.25) (layer F.Cu) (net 10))
 (segment (start 151.13 44.45) (end 149.86 44.45) (width 0.25) (layer F.Cu) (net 10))
 (segment (start 133.35 133.35) (end 136.75 133.35) (width 0.25) (layer F.Cu) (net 6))
 (segment (start 176.53 107.473285) (end 176.53 125.73) (width 0.25) (layer F.Cu) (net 4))
 (segment (start 191.308275 92.69501) (end 176.53 107.473285) (width 0.25) (layer F.Cu) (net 4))
 (segment (start 192.381705 92.69501) (end 191.308275 92.69501) (width 0.25) (layer F.Cu) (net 4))
 (segment (start 193.520019 91.556696) (end 192.381705 92.69501) (width 0.25) (layer F.Cu) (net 4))
 (segment (start 193.520019 81.483304) (end 193.520019 91.556696) (width 0.25) (layer F.Cu) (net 4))
 (segment (start 192.381705 80.34499) (end 193.520019 81.483304) (width 0.25) (layer F.Cu) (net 4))
 (segment (start 138.09501 80.34499) (end 192.381705 80.34499) (width 0.25) (layer F.Cu) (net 4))
 (segment (start 130.81 87.63) (end 138.09501 80.34499) (width 0.25) (layer F.Cu) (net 4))
 (segment (start 130.81 84.23) (end 130.81 87.63) (width 0.25) (layer F.Cu) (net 4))
 (segment (start 120.65 99.148252) (end 112.141758 90.64001) (width 0.25) (layer F.Cu) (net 8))
 (segment (start 120.65 99.92) (end 120.65 99.148252) (width 0.25) (layer F.Cu) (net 8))
 (segment (start 115.785 104.785) (end 120.65 99.92) (width 0.25) (layer F.Cu) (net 8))
 (segment (start 111.07 104.785) (end 115.785 104.785) (width 0.25) (layer F.Cu) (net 8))
 (segment (start 120.65 96.52) (end 120.65 99.92) (width 0.25) (layer F.Cu) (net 8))
 (segment (start 134.62 114.3) (end 135.89 113.03) (width 0.25) (layer F.Cu) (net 5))
 (segment (start 133.35 115.57) (end 135.89 113.03) (width 0.25) (layer F.Cu) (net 5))
 (segment (start 133.35 123.43) (end 133.35 115.57) (width 0.25) (layer F.Cu) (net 5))
 (segment (start 133.35 123.43) (end 136.75 123.43) (width 0.25) (layer F.Cu) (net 5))
 (segment (start 140.97 115.57) (end 142.24 114.3) (width 0.25) (layer F.Cu) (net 13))
 (segment (start 135.89 115.57) (end 140.97 115.57) (width 0.25) (layer F.Cu) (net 13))
 (segment (start 167.64 62.23) (end 170.18 64.77) (width 0.25) (layer F.Cu) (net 13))
 (segment (start 165.1 62.23) (end 167.64 62.23) (width 0.25) (layer F.Cu) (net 13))
 (segment (start 179.76 86.83681) (end 179.76 87.65) (width 0.25) (layer F.Cu) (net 13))
 (segment (start 185.07681 81.52) (end 179.76 86.83681) (width 0.25) (layer F.Cu) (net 13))
 (segment (start 191.77 81.52) (end 185.07681 81.52) (width 0.25) (layer F.Cu) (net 13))
 (segment (start 156.21 91.44) (end 157.48 90.17) (width 0.25) (layer F.Cu) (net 13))
 (segment (start 151.13 91.44) (end 156.21 91.44) (width 0.25) (layer F.Cu) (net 13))
 (segment (start 156.21 104.14) (end 157.48 102.87) (width 0.25) (layer F.Cu) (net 13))
 (segment (start 151.13 104.14) (end 156.21 104.14) (width 0.25) (layer F.Cu) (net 13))
 (segment (start 143.365001 115.425001) (end 142.24 114.3) (width 0.25) (layer F.Cu) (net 13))
 (segment (start 147.860001 115.425001) (end 143.365001 115.425001) (width 0.25) (layer F.Cu) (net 13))
 (segment (start 151.13 112.155002) (end 147.860001 115.425001) (width 0.25) (layer F.Cu) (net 13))
 (segment (start 151.13 104.14) (end 151.13 112.155002) (width 0.25) (layer F.Cu) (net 13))
 (segment (start 152.4 77.47) (end 151.13 78.74) (width 0.25) (layer F.Cu) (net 13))
 (segment (start 157.48 77.47) (end 152.4 77.47) (width 0.25) (layer F.Cu) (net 13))
 (segment (start 149.414999 77.915001) (end 151.13 76.2) (width 0.25) (layer F.Cu) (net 11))
 (segment (start 122.605001 77.915001) (end 149.414999 77.915001) (width 0.25) (layer F.Cu) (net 11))
 (segment (start 120.89 76.2) (end 122.605001 77.915001) (width 0.25) (layer F.Cu) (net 11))
 (segment (start 120.89 76.2) (end 120.89 72.8) (width 0.25) (layer F.Cu) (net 11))
 (segment (start 156.21 73.66) (end 157.48 74.93) (width 0.25) (layer F.Cu) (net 23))
 (segment (start 151.13 73.66) (end 156.21 73.66) (width 0.25) (layer F.Cu) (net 23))
 (segment (start 130.81 72.8) (end 141.38 72.8) (width 0.25) (layer F.Cu) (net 12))
 (segment (start 141.38 72.8) (end 142.24 73.66) (width 0.25) (layer F.Cu) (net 12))
 (segment (start 130.81 76.2) (end 130.81 72.8) (width 0.25) (layer F.Cu) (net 12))
 (via (at 204.47 104.14) (size 0.8) (drill 0.4) (layers F.Cu B.Cu) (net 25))
 (segment (start 170.419492 60.95249) (end 171.65501 62.188008) (width 0.25) (layer F.Cu) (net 22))
 (segment (start 171.65501 62.188008) (end 171.65501 65.448402) (width 0.25) (layer F.Cu) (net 22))
 (segment (start 191.77 84.02) (end 185.62 90.17) (width 0.25) (layer F.Cu) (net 22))
 (segment (start 179.78 90.17) (end 179.76 90.15) (width 0.25) (layer F.Cu) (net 22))
 (segment (start 185.62 90.17) (end 179.78 90.17) (width 0.25) (layer F.Cu) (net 22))
 (segment (start 187.108232 114.925) (end 187.38 114.925) (width 0.25) (layer F.Cu) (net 15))
 (segment (start 186.20499 115.828242) (end 187.108232 114.925) (width 0.25) (layer F.Cu) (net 15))
 (segment (start 186.483242 116.80001) (end 186.20499 116.521758) (width 0.25) (layer F.Cu) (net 15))
 (segment (start 186.20499 116.521758) (end 186.20499 115.828242) (width 0.25) (layer F.Cu) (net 15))
 (segment (start 188.276758 116.80001) (end 186.483242 116.80001) (width 0.25) (layer F.Cu) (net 15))
 (segment (start 192.25501 112.821758) (end 188.276758 116.80001) (width 0.25) (layer F.Cu) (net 15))
 (segment (start 192.25501 97.00501) (end 192.25501 112.821758) (width 0.25) (layer F.Cu) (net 15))
 (segment (start 191.77 96.52) (end 192.25501 97.00501) (width 0.25) (layer F.Cu) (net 15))
 (segment (start 140.97 110.49) (end 142.24 111.76) (width 0.25) (layer F.Cu) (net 20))
 (segment (start 135.89 110.49) (end 140.97 110.49) (width 0.25) (layer F.Cu) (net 20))
 (segment (start 136.915001 109.464999) (end 135.89 110.49) (width 0.25) (layer F.Cu) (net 20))
 (segment (start 144.78 114.3) (end 142.24 111.76) (width 0.25) (layer F.Cu) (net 20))
 (segment (start 147.32 114.3) (end 144.78 114.3) (width 0.25) (layer F.Cu) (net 20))
 (segment (start 169.157002 67.31) (end 165.1 67.31) (width 0.25) (layer F.Cu) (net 21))
 (segment (start 171.205001 65.262001) (end 169.157002 67.31) (width 0.25) (layer F.Cu) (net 21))
 (segment (start 171.205001 63.255001) (end 171.205001 65.262001) (width 0.25) (layer F.Cu) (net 21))
 (segment (start 170.18 62.23) (end 171.205001 63.255001) (width 0.25) (layer F.Cu) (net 21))
 (segment (start 126.8 90.19) (end 111.07 90.19) (width 0.25) (layer F.Cu) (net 21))
 (segment (start 147.32 110.71) (end 126.8 90.19) (width 0.25) (layer F.Cu) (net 21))
 (segment (start 147.32 111.76) (end 147.32 110.71) (width 0.25) (layer F.Cu) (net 21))
 (segment (start 187.651768 116.175) (end 187.38 116.175) (width 0.25) (layer F.Cu) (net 16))
 (segment (start 188.90499 114.921778) (end 187.651768 116.175) (width 0.25) (layer F.Cu) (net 16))
 (segment (start 188.90499 96.88501) (end 188.90499 114.921778) (width 0.25) (layer F.Cu) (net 16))
 (segment (start 191.77 94.02) (end 188.90499 96.88501) (width 0.25) (layer F.Cu) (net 16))
 (segment (start 111.07 78.095) (end 111.07 87.69) (width 0.25) (layer F.Cu) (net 14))
 (segment (start 193.07001 85.21999) (end 191.77 86.52) (width 0.25) (layer F.Cu) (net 14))
 (segment (start 193.07001 83.533295) (end 193.07001 85.21999) (width 0.25) (layer F.Cu) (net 14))
 (segment (start 192.381705 82.84499) (end 193.07001 83.533295) (width 0.25) (layer F.Cu) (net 14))
 (segment (start 191.158295 82.84499) (end 192.381705 82.84499) (width 0.25) (layer F.Cu) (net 14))
 (segment (start 185.103285 88.9) (end 191.158295 82.84499) (width 0.25) (layer F.Cu) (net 14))
 (segment (start 179.76 88.9) (end 185.103285 88.9) (width 0.25) (layer F.Cu) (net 14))
 (segment (start 186.045 113.675) (end 187.38 113.675) (width 0.25) (layer F.Cu) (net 14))
 (segment (start 185.75498 113.96502) (end 186.045 113.675) (width 0.25) (layer F.Cu) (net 14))
 (segment (start 176.876758 126.90501) (end 185.75498 118.026788) (width 0.25) (layer F.Cu) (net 14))
 (segment (start 185.75498 118.026788) (end 185.75498 113.96502) (width 0.25) (layer F.Cu) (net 14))
 (segment (start 175.60501 126.90501) (end 176.876758 126.90501) (width 0.25) (layer F.Cu) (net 14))
 (segment (start 175.28 126.58) (end 175.60501 126.90501) (width 0.25) (layer F.Cu) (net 14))
 (segment (start 175.28 125.73) (end 175.28 126.58) (width 0.25) (layer F.Cu) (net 14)))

